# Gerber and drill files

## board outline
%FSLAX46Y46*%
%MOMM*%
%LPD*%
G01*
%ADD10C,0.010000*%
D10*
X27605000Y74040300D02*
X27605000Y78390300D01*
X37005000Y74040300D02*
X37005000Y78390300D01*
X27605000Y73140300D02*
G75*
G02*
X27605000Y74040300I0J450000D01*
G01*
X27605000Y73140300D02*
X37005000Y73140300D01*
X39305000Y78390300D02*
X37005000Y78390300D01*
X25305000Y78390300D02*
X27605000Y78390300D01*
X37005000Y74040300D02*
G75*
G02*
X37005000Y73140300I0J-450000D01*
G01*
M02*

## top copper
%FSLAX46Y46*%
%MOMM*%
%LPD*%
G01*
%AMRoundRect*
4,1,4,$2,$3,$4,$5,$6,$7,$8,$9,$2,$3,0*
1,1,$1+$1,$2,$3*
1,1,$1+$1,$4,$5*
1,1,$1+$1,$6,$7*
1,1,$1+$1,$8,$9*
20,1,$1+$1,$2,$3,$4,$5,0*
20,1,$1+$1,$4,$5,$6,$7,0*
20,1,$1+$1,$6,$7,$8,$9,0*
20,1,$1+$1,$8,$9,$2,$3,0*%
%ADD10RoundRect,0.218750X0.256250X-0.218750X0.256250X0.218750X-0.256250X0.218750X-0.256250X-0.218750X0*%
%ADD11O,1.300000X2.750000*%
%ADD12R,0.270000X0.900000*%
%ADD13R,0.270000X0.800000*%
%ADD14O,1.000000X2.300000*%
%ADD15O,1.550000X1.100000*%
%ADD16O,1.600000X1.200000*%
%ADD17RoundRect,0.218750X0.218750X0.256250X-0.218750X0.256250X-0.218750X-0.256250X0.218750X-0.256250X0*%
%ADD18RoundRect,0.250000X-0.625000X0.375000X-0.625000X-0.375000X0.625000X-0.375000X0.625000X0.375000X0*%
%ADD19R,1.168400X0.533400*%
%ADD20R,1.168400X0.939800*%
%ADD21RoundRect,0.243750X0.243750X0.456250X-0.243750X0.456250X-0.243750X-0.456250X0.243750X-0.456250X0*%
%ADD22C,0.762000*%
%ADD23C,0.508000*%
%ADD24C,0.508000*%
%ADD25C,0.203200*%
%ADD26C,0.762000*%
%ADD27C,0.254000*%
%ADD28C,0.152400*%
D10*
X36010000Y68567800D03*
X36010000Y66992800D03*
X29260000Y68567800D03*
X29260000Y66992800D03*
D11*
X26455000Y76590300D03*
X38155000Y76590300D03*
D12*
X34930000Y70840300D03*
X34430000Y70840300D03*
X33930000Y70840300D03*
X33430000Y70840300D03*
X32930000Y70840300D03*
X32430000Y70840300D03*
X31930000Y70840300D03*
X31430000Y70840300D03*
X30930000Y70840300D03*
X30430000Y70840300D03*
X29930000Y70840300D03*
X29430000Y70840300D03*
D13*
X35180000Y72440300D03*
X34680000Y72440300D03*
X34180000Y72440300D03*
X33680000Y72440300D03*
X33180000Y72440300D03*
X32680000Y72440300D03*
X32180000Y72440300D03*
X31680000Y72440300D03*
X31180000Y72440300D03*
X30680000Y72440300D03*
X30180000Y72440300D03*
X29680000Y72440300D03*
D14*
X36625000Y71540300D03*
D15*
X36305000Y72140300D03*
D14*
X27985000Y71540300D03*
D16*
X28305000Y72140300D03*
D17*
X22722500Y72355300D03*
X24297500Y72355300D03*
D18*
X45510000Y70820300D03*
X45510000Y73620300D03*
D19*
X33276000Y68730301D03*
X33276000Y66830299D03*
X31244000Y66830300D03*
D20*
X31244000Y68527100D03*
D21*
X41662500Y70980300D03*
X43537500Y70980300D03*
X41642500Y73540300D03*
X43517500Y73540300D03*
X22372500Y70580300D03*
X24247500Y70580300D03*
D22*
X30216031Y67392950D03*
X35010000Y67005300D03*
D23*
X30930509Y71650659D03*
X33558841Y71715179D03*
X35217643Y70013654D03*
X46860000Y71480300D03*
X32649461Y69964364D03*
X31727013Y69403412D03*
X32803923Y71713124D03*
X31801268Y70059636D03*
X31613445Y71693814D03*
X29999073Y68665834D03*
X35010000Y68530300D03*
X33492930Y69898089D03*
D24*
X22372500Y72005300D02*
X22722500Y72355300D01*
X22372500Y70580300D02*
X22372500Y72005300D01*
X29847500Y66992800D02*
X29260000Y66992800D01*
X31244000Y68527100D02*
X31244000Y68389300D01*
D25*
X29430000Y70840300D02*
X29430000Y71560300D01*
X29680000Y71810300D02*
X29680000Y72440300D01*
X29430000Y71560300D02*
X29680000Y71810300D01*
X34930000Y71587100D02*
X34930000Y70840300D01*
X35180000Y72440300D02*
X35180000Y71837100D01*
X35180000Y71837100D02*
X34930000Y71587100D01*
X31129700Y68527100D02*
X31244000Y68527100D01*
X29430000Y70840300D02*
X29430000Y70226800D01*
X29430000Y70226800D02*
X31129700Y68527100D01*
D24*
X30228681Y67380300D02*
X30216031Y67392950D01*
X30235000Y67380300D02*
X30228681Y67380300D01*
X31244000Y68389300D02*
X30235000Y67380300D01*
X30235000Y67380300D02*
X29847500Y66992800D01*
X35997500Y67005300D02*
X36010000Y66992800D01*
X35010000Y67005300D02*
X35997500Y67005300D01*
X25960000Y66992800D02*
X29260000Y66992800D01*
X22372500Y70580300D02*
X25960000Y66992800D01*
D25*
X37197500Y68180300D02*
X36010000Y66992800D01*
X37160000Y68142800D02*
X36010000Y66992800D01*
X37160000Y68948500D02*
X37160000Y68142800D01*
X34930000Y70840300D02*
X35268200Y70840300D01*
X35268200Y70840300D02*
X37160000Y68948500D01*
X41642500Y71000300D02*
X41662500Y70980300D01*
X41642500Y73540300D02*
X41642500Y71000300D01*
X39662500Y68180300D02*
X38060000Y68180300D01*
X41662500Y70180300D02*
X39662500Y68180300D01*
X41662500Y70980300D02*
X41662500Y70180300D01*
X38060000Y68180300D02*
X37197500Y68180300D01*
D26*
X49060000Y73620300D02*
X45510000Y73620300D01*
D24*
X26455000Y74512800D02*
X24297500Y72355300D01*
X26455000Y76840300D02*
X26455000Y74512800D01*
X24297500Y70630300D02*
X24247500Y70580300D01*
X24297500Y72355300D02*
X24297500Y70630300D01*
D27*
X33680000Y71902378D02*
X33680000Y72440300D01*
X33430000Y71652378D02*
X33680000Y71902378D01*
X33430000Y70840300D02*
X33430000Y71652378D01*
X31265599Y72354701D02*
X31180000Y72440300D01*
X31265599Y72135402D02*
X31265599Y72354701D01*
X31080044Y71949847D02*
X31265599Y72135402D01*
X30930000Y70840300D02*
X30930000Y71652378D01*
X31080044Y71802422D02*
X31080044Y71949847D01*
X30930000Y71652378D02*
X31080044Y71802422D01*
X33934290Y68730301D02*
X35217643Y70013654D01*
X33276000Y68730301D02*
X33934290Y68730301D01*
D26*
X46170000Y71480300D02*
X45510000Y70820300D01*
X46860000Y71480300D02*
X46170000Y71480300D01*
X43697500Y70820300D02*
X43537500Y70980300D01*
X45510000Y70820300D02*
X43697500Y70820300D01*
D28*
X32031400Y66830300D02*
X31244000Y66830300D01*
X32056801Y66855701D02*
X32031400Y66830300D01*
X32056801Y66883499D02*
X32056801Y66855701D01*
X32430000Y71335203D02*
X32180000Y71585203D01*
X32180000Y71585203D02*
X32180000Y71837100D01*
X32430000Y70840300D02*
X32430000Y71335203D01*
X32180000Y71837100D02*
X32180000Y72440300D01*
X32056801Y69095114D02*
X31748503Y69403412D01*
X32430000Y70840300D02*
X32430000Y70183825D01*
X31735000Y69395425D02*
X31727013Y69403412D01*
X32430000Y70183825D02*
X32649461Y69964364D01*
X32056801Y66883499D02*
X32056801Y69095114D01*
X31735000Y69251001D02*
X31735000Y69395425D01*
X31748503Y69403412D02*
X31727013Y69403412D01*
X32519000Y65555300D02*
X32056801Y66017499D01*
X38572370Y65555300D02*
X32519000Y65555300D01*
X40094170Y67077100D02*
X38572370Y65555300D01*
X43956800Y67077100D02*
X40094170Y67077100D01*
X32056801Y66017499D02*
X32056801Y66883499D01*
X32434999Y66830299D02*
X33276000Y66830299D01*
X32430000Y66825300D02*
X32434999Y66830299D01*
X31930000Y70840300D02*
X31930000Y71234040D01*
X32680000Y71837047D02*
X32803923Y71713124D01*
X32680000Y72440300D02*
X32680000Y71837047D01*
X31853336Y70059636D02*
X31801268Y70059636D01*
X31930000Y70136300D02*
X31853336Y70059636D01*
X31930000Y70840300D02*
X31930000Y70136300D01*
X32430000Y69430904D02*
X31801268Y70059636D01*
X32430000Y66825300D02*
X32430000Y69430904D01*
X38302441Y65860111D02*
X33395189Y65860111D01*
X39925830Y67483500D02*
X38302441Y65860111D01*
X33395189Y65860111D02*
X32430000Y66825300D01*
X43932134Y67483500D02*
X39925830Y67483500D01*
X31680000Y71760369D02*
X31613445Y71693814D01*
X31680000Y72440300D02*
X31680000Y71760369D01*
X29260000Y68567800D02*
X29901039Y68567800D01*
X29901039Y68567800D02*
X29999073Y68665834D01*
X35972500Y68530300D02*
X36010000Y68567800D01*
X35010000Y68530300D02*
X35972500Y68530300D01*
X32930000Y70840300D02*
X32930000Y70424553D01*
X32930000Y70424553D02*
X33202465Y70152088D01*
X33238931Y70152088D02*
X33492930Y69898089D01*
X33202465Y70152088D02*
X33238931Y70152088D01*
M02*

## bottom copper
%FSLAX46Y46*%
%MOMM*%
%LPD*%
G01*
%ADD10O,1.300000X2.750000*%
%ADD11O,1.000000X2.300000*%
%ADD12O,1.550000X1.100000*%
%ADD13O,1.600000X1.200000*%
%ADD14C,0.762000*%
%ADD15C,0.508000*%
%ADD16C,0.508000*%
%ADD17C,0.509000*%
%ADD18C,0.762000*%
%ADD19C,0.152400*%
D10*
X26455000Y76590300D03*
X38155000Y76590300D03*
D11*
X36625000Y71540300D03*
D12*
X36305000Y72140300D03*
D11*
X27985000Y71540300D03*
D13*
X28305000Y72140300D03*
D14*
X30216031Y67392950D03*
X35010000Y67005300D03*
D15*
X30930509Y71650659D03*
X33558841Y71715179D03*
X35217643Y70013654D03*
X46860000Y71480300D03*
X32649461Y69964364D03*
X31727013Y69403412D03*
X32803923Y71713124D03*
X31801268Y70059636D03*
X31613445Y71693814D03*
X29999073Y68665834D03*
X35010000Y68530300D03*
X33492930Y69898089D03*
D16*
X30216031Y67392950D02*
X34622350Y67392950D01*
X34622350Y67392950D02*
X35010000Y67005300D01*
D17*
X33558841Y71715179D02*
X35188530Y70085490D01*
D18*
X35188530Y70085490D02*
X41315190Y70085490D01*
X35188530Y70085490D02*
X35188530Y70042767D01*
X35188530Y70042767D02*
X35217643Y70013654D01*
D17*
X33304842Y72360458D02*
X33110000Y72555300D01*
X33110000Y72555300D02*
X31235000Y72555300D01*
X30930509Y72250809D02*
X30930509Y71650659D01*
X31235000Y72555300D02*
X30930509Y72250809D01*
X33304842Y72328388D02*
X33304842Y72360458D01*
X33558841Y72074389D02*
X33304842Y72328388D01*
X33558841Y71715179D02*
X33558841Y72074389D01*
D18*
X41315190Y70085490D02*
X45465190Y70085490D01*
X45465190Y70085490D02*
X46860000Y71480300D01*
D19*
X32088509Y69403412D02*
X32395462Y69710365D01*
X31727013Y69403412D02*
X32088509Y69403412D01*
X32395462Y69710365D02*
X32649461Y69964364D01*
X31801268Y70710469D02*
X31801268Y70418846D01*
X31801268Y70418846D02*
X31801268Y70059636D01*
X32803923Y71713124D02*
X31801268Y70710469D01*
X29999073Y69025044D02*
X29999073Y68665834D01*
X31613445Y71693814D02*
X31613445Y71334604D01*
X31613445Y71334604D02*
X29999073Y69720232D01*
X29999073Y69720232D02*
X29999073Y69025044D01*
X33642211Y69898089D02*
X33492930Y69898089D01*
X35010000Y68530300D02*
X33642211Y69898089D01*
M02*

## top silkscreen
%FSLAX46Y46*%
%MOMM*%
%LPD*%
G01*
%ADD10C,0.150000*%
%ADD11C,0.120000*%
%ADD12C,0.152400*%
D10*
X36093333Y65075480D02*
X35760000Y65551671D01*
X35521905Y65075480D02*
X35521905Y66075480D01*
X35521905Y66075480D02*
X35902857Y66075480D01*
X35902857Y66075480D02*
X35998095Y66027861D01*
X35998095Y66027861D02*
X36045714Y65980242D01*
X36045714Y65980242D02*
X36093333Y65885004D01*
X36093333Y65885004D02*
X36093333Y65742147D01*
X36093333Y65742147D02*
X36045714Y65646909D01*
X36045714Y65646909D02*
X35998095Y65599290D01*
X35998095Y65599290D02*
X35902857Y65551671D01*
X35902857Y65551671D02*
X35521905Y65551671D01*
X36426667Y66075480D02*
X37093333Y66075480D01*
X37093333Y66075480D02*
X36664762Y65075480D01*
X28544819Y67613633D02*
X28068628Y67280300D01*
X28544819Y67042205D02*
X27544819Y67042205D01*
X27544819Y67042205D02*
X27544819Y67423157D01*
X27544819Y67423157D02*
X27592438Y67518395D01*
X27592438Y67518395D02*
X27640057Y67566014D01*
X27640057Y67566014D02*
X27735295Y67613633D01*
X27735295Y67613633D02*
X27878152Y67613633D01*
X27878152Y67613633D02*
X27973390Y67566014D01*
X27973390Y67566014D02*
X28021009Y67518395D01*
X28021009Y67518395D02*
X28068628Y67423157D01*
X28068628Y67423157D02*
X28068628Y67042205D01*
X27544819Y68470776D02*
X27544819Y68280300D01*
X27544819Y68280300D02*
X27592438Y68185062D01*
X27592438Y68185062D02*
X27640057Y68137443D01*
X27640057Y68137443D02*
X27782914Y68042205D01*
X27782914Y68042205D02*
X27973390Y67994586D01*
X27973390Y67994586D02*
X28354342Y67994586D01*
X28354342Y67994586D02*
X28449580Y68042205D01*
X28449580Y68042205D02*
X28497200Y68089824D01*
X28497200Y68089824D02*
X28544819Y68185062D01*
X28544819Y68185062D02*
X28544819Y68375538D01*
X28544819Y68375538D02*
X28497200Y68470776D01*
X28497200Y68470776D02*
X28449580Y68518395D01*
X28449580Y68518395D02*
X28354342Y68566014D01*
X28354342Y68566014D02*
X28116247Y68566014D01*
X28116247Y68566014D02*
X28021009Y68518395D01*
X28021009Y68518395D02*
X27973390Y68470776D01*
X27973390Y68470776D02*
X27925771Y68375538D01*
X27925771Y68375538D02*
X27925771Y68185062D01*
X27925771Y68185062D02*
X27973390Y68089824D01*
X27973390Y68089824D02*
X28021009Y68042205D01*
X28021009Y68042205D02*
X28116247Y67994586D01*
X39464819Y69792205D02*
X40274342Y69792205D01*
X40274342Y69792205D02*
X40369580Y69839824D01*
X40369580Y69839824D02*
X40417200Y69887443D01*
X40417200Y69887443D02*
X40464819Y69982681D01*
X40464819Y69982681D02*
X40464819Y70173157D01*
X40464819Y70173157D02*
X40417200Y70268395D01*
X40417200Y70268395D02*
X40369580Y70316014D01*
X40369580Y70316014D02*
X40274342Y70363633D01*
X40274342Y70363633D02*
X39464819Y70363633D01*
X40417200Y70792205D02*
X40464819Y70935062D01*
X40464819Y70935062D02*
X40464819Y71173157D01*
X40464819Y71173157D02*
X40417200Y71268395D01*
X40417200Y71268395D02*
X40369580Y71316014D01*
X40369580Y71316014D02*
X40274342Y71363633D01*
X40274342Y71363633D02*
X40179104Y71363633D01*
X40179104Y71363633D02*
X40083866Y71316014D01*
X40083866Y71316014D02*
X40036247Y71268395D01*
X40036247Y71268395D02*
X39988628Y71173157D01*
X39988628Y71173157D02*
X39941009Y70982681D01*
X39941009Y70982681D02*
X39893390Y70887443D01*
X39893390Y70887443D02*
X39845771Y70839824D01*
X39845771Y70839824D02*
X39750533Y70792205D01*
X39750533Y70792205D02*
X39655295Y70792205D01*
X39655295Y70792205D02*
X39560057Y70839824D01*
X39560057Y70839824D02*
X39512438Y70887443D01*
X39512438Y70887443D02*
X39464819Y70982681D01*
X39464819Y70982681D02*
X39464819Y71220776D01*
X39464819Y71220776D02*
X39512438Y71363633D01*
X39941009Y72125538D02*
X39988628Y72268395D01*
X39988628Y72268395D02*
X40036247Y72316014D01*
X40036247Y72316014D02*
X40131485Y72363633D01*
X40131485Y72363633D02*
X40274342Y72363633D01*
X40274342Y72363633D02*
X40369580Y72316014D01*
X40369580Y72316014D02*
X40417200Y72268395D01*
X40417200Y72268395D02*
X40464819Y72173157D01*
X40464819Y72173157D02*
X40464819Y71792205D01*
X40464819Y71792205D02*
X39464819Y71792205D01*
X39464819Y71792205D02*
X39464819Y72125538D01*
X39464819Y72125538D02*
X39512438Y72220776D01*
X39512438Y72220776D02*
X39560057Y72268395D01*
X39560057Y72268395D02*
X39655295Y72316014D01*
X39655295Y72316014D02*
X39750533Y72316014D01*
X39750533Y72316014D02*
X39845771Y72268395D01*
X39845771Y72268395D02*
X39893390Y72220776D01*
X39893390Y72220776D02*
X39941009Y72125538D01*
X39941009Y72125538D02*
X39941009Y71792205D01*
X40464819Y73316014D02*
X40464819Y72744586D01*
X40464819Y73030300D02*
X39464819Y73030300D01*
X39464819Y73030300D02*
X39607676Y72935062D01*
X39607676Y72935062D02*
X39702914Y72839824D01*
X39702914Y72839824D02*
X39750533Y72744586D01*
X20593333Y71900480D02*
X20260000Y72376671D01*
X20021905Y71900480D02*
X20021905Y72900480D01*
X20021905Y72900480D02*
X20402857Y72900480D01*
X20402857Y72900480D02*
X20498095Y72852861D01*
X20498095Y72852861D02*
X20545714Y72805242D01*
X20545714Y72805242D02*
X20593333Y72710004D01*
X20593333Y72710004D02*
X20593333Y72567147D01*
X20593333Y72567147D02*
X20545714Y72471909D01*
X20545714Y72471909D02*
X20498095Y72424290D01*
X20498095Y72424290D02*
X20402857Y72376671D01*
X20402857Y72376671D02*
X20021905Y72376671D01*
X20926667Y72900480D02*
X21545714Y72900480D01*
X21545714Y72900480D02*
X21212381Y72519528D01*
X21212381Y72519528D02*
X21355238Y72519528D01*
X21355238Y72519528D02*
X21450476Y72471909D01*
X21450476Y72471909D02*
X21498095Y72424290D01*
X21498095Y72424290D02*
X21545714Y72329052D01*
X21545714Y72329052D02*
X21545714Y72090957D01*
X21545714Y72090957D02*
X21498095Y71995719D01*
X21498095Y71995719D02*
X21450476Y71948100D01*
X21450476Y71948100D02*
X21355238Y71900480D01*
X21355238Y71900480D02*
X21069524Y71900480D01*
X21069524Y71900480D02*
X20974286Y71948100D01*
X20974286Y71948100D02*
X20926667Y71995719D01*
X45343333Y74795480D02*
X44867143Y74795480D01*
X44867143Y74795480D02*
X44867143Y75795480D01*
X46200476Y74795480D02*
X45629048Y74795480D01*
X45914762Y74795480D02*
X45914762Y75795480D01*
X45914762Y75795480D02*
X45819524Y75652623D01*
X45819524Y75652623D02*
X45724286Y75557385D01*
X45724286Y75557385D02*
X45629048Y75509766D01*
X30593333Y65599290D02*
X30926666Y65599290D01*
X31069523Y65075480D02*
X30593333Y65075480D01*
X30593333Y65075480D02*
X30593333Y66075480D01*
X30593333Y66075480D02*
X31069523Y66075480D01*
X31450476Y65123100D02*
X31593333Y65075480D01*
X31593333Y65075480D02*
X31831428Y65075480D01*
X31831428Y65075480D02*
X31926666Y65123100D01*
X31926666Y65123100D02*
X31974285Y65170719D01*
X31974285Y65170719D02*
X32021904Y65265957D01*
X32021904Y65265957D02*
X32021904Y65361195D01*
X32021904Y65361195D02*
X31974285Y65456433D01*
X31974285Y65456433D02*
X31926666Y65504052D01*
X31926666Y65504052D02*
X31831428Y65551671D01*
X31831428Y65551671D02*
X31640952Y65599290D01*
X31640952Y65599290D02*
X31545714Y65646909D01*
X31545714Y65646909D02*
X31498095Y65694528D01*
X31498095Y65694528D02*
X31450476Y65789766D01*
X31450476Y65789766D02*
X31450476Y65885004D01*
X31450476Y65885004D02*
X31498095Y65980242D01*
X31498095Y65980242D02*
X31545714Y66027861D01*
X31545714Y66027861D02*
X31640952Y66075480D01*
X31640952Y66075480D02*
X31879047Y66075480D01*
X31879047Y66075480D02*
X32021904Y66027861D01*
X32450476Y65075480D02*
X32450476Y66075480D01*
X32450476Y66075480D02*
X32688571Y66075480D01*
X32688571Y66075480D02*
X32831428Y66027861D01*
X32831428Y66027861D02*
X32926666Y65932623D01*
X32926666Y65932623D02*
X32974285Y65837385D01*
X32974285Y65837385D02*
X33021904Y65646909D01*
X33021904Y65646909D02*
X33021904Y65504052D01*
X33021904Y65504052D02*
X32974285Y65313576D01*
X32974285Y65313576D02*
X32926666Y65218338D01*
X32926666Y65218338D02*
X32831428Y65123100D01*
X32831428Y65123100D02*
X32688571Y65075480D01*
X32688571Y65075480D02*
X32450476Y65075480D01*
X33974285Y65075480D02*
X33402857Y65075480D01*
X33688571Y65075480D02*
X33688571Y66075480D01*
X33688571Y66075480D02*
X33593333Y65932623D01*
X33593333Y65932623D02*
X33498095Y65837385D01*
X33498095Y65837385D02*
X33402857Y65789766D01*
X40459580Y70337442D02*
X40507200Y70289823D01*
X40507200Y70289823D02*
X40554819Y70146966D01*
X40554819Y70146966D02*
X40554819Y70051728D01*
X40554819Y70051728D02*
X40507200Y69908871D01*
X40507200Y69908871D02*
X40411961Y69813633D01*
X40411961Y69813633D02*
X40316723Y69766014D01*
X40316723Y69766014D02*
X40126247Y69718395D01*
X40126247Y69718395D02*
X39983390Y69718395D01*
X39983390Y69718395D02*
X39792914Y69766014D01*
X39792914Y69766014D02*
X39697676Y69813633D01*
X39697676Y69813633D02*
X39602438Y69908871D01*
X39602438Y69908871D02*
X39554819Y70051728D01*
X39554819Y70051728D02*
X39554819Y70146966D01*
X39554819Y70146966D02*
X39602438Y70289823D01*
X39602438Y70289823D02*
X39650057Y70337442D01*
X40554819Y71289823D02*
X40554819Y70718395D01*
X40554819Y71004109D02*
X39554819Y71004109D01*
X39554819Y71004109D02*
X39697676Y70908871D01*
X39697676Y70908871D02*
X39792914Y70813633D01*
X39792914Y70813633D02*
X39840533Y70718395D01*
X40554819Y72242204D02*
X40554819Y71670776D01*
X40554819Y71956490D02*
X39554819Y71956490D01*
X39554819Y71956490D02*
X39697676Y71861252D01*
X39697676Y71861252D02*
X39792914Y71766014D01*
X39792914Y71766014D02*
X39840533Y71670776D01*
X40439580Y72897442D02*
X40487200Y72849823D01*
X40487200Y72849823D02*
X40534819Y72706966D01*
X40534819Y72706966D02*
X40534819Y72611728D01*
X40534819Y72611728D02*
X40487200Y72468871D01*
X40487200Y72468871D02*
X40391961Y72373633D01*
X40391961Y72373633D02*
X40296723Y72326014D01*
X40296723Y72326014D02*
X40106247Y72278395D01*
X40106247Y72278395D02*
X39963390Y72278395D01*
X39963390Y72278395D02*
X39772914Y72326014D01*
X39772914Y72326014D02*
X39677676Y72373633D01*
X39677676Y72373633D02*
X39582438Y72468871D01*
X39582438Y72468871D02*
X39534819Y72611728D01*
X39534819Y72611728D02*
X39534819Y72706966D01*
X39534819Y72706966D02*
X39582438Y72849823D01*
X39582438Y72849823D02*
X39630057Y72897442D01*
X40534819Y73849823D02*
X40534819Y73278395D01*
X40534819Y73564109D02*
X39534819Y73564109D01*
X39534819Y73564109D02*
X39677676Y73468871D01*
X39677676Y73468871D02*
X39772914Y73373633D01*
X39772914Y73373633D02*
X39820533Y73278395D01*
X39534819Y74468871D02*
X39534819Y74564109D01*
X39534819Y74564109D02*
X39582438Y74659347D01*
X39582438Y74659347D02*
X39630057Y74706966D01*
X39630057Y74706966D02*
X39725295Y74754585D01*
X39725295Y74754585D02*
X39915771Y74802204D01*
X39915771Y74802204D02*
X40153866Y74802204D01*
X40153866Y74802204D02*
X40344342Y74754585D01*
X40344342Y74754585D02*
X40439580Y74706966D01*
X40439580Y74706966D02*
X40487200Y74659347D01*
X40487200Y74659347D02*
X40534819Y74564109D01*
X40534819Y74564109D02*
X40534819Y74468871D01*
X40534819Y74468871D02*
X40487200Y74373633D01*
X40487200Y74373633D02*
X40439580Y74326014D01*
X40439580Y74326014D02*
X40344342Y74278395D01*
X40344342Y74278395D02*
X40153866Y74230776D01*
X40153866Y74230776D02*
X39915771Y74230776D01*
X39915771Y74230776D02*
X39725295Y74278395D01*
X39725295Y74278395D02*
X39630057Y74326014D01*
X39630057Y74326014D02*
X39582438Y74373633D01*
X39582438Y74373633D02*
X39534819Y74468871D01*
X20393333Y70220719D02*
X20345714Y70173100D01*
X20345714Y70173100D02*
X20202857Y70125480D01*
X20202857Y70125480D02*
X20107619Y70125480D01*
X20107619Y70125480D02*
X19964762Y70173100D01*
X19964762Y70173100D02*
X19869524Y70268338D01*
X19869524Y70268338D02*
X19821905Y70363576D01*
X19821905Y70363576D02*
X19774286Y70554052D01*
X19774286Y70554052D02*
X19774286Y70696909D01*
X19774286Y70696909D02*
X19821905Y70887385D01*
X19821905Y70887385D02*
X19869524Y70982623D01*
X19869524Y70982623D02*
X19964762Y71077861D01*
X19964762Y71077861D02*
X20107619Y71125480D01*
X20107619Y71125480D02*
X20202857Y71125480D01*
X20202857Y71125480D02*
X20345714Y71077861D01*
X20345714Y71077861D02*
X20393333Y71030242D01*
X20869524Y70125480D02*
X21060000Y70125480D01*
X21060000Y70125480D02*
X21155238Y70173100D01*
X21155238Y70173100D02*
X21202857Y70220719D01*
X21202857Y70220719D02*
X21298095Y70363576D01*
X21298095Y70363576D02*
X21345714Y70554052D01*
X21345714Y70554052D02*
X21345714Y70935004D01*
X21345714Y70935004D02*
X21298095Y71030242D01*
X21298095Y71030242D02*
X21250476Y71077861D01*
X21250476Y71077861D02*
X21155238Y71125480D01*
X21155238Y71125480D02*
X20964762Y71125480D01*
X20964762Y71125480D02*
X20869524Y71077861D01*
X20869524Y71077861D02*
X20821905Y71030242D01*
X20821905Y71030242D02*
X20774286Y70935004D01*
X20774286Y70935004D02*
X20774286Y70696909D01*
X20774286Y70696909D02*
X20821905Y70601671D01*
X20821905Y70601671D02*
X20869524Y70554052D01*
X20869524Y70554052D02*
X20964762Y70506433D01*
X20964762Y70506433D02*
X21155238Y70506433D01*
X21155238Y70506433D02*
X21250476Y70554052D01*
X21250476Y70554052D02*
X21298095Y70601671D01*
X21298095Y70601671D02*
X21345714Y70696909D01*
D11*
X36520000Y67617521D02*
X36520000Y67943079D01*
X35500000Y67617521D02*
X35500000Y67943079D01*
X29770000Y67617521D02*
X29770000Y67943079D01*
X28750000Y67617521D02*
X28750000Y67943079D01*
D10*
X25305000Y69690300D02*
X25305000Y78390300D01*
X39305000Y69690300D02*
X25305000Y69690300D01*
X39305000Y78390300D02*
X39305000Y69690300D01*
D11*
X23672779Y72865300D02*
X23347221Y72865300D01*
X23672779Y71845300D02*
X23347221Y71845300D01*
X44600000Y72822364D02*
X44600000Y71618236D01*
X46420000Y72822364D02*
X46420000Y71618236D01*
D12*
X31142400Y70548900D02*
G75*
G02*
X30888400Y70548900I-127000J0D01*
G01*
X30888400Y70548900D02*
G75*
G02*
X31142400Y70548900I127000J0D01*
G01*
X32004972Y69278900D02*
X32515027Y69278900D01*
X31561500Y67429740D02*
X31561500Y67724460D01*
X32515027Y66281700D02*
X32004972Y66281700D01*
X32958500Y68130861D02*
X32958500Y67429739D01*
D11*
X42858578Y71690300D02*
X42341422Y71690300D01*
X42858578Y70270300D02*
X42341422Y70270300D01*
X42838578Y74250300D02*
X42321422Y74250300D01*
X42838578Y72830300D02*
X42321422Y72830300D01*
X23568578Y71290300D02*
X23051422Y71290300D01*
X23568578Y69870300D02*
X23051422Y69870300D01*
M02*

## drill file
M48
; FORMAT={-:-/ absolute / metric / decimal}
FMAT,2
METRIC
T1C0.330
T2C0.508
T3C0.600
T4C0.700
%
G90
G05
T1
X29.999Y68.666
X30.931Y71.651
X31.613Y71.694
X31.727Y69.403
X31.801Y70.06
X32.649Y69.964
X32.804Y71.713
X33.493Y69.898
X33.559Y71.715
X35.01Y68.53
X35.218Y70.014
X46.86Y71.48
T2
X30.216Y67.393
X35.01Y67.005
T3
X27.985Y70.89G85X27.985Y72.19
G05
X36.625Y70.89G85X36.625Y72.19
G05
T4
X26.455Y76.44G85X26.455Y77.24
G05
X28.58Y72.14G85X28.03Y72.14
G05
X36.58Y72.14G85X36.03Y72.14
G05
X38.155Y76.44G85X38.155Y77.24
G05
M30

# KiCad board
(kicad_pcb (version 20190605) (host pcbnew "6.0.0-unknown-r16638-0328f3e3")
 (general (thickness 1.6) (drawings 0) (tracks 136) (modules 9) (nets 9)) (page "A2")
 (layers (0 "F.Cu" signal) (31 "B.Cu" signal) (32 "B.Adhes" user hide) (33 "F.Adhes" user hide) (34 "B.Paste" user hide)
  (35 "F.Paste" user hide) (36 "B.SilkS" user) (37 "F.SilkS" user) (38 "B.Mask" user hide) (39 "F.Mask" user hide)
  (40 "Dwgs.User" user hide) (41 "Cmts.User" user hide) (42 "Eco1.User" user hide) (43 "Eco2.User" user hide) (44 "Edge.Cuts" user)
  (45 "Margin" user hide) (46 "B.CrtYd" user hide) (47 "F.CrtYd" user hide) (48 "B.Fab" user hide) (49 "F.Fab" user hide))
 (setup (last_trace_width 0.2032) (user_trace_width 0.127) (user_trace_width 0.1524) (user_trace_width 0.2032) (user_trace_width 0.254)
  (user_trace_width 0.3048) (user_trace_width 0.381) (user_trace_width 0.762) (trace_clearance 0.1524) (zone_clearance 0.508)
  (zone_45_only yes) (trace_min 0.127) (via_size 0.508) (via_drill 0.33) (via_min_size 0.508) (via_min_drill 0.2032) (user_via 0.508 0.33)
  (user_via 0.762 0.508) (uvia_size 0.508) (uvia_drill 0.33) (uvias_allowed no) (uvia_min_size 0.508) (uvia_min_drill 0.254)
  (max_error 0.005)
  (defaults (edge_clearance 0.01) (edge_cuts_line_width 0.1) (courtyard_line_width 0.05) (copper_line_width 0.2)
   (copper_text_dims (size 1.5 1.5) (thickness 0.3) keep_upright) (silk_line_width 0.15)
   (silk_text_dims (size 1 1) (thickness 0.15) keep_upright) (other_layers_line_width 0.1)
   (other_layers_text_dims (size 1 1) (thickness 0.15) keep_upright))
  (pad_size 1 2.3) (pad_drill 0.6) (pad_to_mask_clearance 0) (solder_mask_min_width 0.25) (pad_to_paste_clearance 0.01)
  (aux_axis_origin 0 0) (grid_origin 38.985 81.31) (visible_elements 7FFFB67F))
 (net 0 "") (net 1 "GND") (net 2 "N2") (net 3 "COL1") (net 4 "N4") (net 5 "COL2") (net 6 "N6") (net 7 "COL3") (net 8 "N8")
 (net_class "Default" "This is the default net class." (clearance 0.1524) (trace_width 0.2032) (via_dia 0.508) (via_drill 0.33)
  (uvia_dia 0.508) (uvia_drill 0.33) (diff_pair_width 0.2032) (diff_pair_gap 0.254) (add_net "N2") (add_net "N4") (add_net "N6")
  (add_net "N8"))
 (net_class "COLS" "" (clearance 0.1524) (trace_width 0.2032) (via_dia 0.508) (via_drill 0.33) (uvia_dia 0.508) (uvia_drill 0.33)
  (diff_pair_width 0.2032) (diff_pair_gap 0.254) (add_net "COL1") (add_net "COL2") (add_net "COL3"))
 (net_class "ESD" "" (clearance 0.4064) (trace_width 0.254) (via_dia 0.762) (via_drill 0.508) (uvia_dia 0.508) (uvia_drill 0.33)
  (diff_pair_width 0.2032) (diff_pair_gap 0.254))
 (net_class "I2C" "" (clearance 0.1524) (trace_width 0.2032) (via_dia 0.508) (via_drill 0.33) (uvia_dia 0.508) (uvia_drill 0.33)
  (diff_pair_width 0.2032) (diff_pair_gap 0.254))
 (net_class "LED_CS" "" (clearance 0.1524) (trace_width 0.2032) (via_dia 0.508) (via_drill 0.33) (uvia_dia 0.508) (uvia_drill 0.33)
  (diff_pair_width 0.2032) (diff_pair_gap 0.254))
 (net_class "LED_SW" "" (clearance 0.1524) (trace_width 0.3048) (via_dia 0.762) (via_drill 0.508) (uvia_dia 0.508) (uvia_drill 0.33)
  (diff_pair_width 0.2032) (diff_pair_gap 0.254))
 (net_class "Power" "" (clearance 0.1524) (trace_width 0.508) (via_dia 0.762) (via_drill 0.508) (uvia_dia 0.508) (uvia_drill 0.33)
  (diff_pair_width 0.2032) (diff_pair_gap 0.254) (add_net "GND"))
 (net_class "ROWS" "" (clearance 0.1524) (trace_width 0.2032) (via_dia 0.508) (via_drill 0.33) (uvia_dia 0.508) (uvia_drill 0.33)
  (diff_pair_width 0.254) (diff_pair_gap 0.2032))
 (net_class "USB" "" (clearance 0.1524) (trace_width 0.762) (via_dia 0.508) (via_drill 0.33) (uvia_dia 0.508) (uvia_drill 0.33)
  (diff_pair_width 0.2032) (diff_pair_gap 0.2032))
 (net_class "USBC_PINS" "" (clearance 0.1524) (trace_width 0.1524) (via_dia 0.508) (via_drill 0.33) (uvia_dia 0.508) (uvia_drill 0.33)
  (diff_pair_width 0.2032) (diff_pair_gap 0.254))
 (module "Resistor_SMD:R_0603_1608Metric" (layer "F.Cu") (at 36.01 -67.7803 90)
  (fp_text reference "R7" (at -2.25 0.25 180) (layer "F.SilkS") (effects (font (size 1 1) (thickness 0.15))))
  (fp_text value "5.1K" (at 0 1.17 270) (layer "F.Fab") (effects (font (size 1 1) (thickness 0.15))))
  (fp_line (start -0.162779 0.51) (end 0.162779 0.51) (layer "F.SilkS") (width 0.12))
  (fp_line (start -0.162779 -0.51) (end 0.162779 -0.51) (layer "F.SilkS") (width 0.12))
  (pad "2" smd roundrect (at 0.7875 0 90) (size 0.875 0.95) (layers "F.Cu" "F.Paste" "F.Mask") (roundrect_rratio 0.25))
  (pad "1" smd roundrect (at -0.7875 0 90) (size 0.875 0.95) (layers "F.Cu" "F.Paste" "F.Mask") (roundrect_rratio 0.25)))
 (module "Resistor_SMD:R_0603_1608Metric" (layer "F.Cu") (at 29.26 -67.7803 90)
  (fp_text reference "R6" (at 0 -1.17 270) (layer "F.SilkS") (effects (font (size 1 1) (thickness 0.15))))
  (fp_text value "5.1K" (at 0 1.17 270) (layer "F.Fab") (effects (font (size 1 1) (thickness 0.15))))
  (fp_line (start -0.162779 0.51) (end 0.162779 0.51) (layer "F.SilkS") (width 0.12))
  (fp_line (start -0.162779 -0.51) (end 0.162779 -0.51) (layer "F.SilkS") (width 0.12))
  (pad "2" smd roundrect (at 0.7875 0 90) (size 0.875 0.95) (layers "F.Cu" "F.Paste" "F.Mask") (roundrect_rratio 0.25))
  (pad "1" smd roundrect (at -0.7875 0 90) (size 0.875 0.95) (layers "F.Cu" "F.Paste" "F.Mask") (roundrect_rratio 0.25)))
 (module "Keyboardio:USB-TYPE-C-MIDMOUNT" (layer "F.Cu") (at 32.305 -71.5403 180) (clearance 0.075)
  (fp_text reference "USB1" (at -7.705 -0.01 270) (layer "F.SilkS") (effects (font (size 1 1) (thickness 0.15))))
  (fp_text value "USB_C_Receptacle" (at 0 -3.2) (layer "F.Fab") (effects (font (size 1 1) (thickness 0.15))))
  (fp_line (start 7 -1.85) (end 7 6.85) (layer "F.SilkS") (width 0.15))
  (fp_line (start -7 -1.85) (end 7 -1.85) (layer "F.SilkS") (width 0.15))
  (fp_line (start -7 6.85) (end -7 -1.85) (layer "F.SilkS") (width 0.15))
  (fp_line (start 4.7 2.5) (end 4.7 6.85) (layer "Edge.Cuts") (width 0.01))
  (fp_line (start -4.7 2.5) (end -4.7 6.85) (layer "Edge.Cuts") (width 0.01))
  (fp_arc (start 4.7 2.05) (end 4.7 1.6) (angle 180) (layer "Edge.Cuts") (width 0.01))
  (fp_line (start 4.7 1.6) (end -4.7 1.6) (layer "Edge.Cuts") (width 0.01))
  (fp_line (start -7 6.85) (end -4.7 6.85) (layer "Edge.Cuts") (width 0.01))
  (fp_line (start 7 6.85) (end 4.7 6.85) (layer "Edge.Cuts") (width 0.01))
  (fp_arc (start -4.7 2.05) (end -4.7 2.5) (angle 180) (layer "Edge.Cuts") (width 0.01))
  (pad "S1" thru_hole oval (at 5.85 5.3 180) (size 1.3 2.75) (drill oval 0.7 1.5 (offset 0 -0.25)) (layers *.Cu *.Mask))
  (pad "S1" thru_hole oval (at -5.85 5.3 180) (size 1.3 2.75) (drill oval 0.7 1.5 (offset 0 -0.25)) (layers *.Cu *.Mask))
  (pad "A1" smd rect (at -2.625 -0.7 180) (size 0.27 0.9) (layers "F.Cu" "F.Paste" "F.Mask"))
  (pad "A2" smd rect (at -2.125 -0.7 180) (size 0.27 0.9) (layers "F.Cu" "F.Paste" "F.Mask"))
  (pad "A3" smd rect (at -1.625 -0.7 180) (size 0.27 0.9) (layers "F.Cu" "F.Paste" "F.Mask"))
  (pad "A4" smd rect (at -1.125 -0.7 180) (size 0.27 0.9) (layers "F.Cu" "F.Paste" "F.Mask"))
  (pad "A5" smd rect (at -0.625 -0.7 180) (size 0.27 0.9) (layers "F.Cu" "F.Paste" "F.Mask"))
  (pad "A6" smd rect (at -0.125 -0.7 180) (size 0.27 0.9) (layers "F.Cu" "F.Paste" "F.Mask"))
  (pad "A7" smd rect (at 0.375 -0.7 180) (size 0.27 0.9) (layers "F.Cu" "F.Paste" "F.Mask"))
  (pad "A8" smd rect (at 0.875 -0.7 180) (size 0.27 0.9) (layers "F.Cu" "F.Paste" "F.Mask"))
  (pad "A9" smd rect (at 1.375 -0.7 180) (size 0.27 0.9) (layers "F.Cu" "F.Paste" "F.Mask"))
  (pad "A10" smd rect (at 1.875 -0.7 180) (size 0.27 0.9) (layers "F.Cu" "F.Paste" "F.Mask"))
  (pad "A11" smd rect (at 2.375 -0.7 180) (size 0.27 0.9) (layers "F.Cu" "F.Paste" "F.Mask"))
  (pad "A12" smd rect (at 2.875 -0.7 180) (size 0.27 0.9) (layers "F.Cu" "F.Adhes" "F.Paste" "F.Mask"))
  (pad "B12" smd rect (at -2.875 0.9 180) (size 0.27 0.8) (layers "F.Cu" "F.Paste" "F.Mask"))
  (pad "B11" smd rect (at -2.375 0.9 180) (size 0.27 0.8) (layers "F.Cu" "F.Paste" "F.Mask"))
  (pad "B10" smd rect (at -1.875 0.9 180) (size 0.27 0.8) (layers "F.Cu" "F.Paste" "F.Mask"))
  (pad "B9" smd rect (at -1.375 0.9 180) (size 0.27 0.8) (layers "F.Cu" "F.Paste" "F.Mask"))
  (pad "B8" smd rect (at -0.875 0.9 180) (size 0.27 0.8) (layers "F.Cu" "F.Paste" "F.Mask"))
  (pad "B7" smd rect (at -0.375 0.9 180) (size 0.27 0.8) (layers "F.Cu" "F.Paste" "F.Mask"))
  (pad "B6" smd rect (at 0.125 0.9 180) (size 0.27 0.8) (layers "F.Cu" "F.Paste" "F.Mask"))
  (pad "B5" smd rect (at 0.625 0.9 180) (size 0.27 0.8) (layers "F.Cu" "F.Paste" "F.Mask"))
  (pad "B4" smd rect (at 1.125 0.9 180) (size 0.27 0.8) (layers "F.Cu" "F.Paste" "F.Mask"))
  (pad "B3" smd rect (at 1.625 0.9 180) (size 0.27 0.8) (layers "F.Cu" "F.Paste" "F.Mask"))
  (pad "B2" smd rect (at 2.125 0.9 180) (size 0.27 0.8) (layers "F.Cu" "F.Paste" "F.Mask"))
  (pad "B1" smd rect (at 2.625 0.9 180) (size 0.27 0.8) (layers "F.Cu" "F.Paste" "F.Mask"))
  (pad "S1" thru_hole oval (at -4.32 0 180) (size 1 2.3) (drill oval 0.6 1.9) (layers *.Cu *.Mask))
  (pad "S1" thru_hole oval (at -4 0.6 180) (size 1.55 1.1) (drill oval 1.25 0.7) (layers *.Cu *.Mask))
  (pad "S1" thru_hole oval (at 4.32 0 180) (size 1 2.3) (drill oval 0.6 1.9) (layers *.Cu *.Mask))
  (pad "S1" thru_hole oval (at 4 0.6 180) (size 1.6 1.2) (drill oval 1.25 0.7) (layers *.Cu *.Mask)))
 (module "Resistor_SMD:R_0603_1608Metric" (layer "F.Cu") (at 23.51 -72.3553 180)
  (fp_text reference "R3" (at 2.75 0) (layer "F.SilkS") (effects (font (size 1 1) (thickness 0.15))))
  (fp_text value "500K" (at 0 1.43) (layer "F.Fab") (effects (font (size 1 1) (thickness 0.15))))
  (fp_line (start -0.162779 0.51) (end 0.162779 0.51) (layer "F.SilkS") (width 0.12))
  (fp_line (start -0.162779 -0.51) (end 0.162779 -0.51) (layer "F.SilkS") (width 0.12))
  (pad "2" smd roundrect (at 0.7875 0 180) (size 0.875 0.95) (layers "F.Cu" "F.Paste" "F.Mask") (roundrect_rratio 0.25))
  (pad "1" smd roundrect (at -0.7875 0 180) (size 0.875 0.95) (layers "F.Cu" "F.Paste" "F.Mask") (roundrect_rratio 0.25)))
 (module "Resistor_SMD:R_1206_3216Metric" (layer "F.Cu") (at 45.51 -72.2203 270)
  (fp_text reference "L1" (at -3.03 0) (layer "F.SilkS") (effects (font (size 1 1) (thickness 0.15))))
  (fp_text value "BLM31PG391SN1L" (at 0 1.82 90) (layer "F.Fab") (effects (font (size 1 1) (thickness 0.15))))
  (fp_line (start -0.602064 0.91) (end 0.602064 0.91) (layer "F.SilkS") (width 0.12))
  (fp_line (start -0.602064 -0.91) (end 0.602064 -0.91) (layer "F.SilkS") (width 0.12))
  (pad "2" smd roundrect (at 1.4 0 270) (size 1.25 1.75) (layers "F.Cu" "F.Paste" "F.Mask") (roundrect_rratio 0.2))
  (pad "1" smd roundrect (at -1.4 0 270) (size 1.25 1.75) (layers "F.Cu" "F.Paste" "F.Mask") (roundrect_rratio 0.2)))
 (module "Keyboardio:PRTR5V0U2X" (layer "F.Cu") (at 32.26 -67.7803 270)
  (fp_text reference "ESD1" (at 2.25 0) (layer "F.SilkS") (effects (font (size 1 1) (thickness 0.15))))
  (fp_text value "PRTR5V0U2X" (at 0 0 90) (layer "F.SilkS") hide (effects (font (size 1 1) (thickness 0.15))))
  (fp_circle (center -2.7686 1.2446) (end -2.6416 1.2446) (layer "F.SilkS") (width 0.1524))
  (fp_line (start -1.4986 0.255028) (end -1.4986 -0.255027) (layer "F.SilkS") (width 0.1524))
  (fp_line (start 0.35056 0.6985) (end 0.05584 0.6985) (layer "F.SilkS") (width 0.1524))
  (fp_line (start 1.4986 -0.255027) (end 1.4986 0.255028) (layer "F.SilkS") (width 0.1524))
  (fp_line (start -0.350561 -0.6985) (end 0.350561 -0.6985) (layer "F.SilkS") (width 0.1524))
  (pad "4" smd rect (at -0.950001 -1.016 270) (size 0.5334 1.1684) (layers "F.Cu" "F.Paste" "F.Mask"))
  (pad "3" smd rect (at 0.950001 -1.016 270) (size 0.5334 1.1684) (layers "F.Cu" "F.Paste" "F.Mask"))
  (pad "2" smd rect (at 0.95 1.016 270) (size 0.5334 1.1684) (layers "F.Cu" "F.Paste" "F.Mask"))
  (pad "1" smd rect (at -0.7468 1.016 270) (size 0.9398 1.1684) (layers "F.Cu" "F.Paste" "F.Mask")))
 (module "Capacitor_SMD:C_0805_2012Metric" (layer "F.Cu") (at 42.6 -70.9803 180)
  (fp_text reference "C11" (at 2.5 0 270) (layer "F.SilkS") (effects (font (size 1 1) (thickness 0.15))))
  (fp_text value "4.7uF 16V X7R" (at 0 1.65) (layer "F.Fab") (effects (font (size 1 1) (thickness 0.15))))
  (fp_line (start -0.258578 0.71) (end 0.258578 0.71) (layer "F.SilkS") (width 0.12))
  (fp_line (start -0.258578 -0.71) (end 0.258578 -0.71) (layer "F.SilkS") (width 0.12))
  (pad "2" smd roundrect (at 0.9375 0 180) (size 0.975 1.4) (layers "F.Cu" "F.Paste" "F.Mask") (roundrect_rratio 0.25))
  (pad "1" smd roundrect (at -0.9375 0 180) (size 0.975 1.4) (layers "F.Cu" "F.Paste" "F.Mask") (roundrect_rratio 0.25)))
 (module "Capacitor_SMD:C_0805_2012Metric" (layer "F.Cu") (at 42.58 -73.5403 180)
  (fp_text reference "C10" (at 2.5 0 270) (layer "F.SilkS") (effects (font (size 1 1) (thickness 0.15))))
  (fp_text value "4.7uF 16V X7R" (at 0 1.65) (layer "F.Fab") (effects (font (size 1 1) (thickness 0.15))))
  (fp_line (start -0.258578 0.71) (end 0.258578 0.71) (layer "F.SilkS") (width 0.12))
  (fp_line (start -0.258578 -0.71) (end 0.258578 -0.71) (layer "F.SilkS") (width 0.12))
  (pad "2" smd roundrect (at 0.9375 0 180) (size 0.975 1.4) (layers "F.Cu" "F.Paste" "F.Mask") (roundrect_rratio 0.25))
  (pad "1" smd roundrect (at -0.9375 0 180) (size 0.975 1.4) (layers "F.Cu" "F.Paste" "F.Mask") (roundrect_rratio 0.25)))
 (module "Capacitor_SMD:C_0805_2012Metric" (layer "F.Cu") (at 23.31 -70.5803 180)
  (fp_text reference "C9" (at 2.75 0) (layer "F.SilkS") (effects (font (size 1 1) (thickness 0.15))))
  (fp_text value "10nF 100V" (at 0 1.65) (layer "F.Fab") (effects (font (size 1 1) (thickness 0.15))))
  (fp_line (start -0.258578 0.71) (end 0.258578 0.71) (layer "F.SilkS") (width 0.12))
  (fp_line (start -0.258578 -0.71) (end 0.258578 -0.71) (layer "F.SilkS") (width 0.12))
  (pad "2" smd roundrect (at 0.9375 0 180) (size 0.975 1.4) (layers "F.Cu" "F.Paste" "F.Mask") (roundrect_rratio 0.25))
  (pad "1" smd roundrect (at -0.9375 0 180) (size 0.975 1.4) (layers "F.Cu" "F.Paste" "F.Mask") (roundrect_rratio 0.25)))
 (segment (start 22.3725 -72.0053) (end 22.7225 -72.3553) (width 0.508) (layer "F.Cu") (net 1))
 (segment (start 22.3725 -70.5803) (end 22.3725 -72.0053) (width 0.508) (layer "F.Cu") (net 1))
 (segment (start 29.8475 -66.9928) (end 29.26 -66.9928) (width 0.508) (layer "F.Cu") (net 1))
 (segment (start 31.244 -68.5271) (end 31.244 -68.3893) (width 0.508) (layer "F.Cu") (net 1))
 (segment (start 29.43 -70.8403) (end 29.43 -71.5603) (width 0.2032) (layer "F.Cu") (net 1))
 (segment (start 29.68 -71.8103) (end 29.68 -72.4403) (width 0.2032) (layer "F.Cu") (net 1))
 (segment (start 29.43 -71.5603) (end 29.68 -71.8103) (width 0.2032) (layer "F.Cu") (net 1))
 (segment (start 34.93 -71.5871) (end 34.93 -70.8403) (width 0.2032) (layer "F.Cu") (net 1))
 (segment (start 35.18 -72.4403) (end 35.18 -71.8371) (width 0.2032) (layer "F.Cu") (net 1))
 (segment (start 35.18 -71.8371) (end 34.93 -71.5871) (width 0.2032) (layer "F.Cu") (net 1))
 (segment (start 31.1297 -68.5271) (end 31.244 -68.5271) (width 0.2032) (layer "F.Cu") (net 1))
 (segment (start 29.43 -70.8403) (end 29.43 -70.2268) (width 0.2032) (layer "F.Cu") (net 1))
 (segment (start 29.43 -70.2268) (end 31.1297 -68.5271) (width 0.2032) (layer "F.Cu") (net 1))
 (via (at 30.216031 -67.39295) (size 0.762) (drill 0.508) (layers "F.Cu" "B.Cu") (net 1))
 (segment (start 30.228681 -67.3803) (end 30.216031 -67.39295) (width 0.508) (layer "F.Cu") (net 1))
 (segment (start 30.235 -67.3803) (end 30.228681 -67.3803) (width 0.508) (layer "F.Cu") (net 1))
 (segment (start 31.244 -68.3893) (end 30.235 -67.3803) (width 0.508) (layer "F.Cu") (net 1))
 (segment (start 30.235 -67.3803) (end 29.8475 -66.9928) (width 0.508) (layer "F.Cu") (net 1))
 (via (at 35.01 -67.0053) (size 0.762) (drill 0.508) (layers "F.Cu" "B.Cu") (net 1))
 (segment (start 30.216031 -67.39295) (end 34.62235 -67.39295) (width 0.508) (layer "B.Cu") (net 1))
 (segment (start 34.62235 -67.39295) (end 35.01 -67.0053) (width 0.508) (layer "B.Cu") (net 1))
 (segment (start 35.9975 -67.0053) (end 36.01 -66.9928) (width 0.508) (layer "F.Cu") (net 1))
 (segment (start 35.01 -67.0053) (end 35.9975 -67.0053) (width 0.508) (layer "F.Cu") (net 1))
 (segment (start 25.96 -66.9928) (end 29.26 -66.9928) (width 0.508) (layer "F.Cu") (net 1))
 (segment (start 22.3725 -70.5803) (end 25.96 -66.9928) (width 0.508) (layer "F.Cu") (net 1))
 (segment (start 37.1975 -68.1803) (end 36.01 -66.9928) (width 0.2032) (layer "F.Cu") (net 1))
 (segment (start 37.16 -68.1428) (end 36.01 -66.9928) (width 0.2032) (layer "F.Cu") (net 1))
 (segment (start 37.16 -68.9485) (end 37.16 -68.1428) (width 0.2032) (layer "F.Cu") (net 1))
 (segment (start 34.93 -70.8403) (end 35.2682 -70.8403) (width 0.2032) (layer "F.Cu") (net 1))
 (segment (start 35.2682 -70.8403) (end 37.16 -68.9485) (width 0.2032) (layer "F.Cu") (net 1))
 (segment (start 41.6425 -71.0003) (end 41.6625 -70.9803) (width 0.2032) (layer "F.Cu") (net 1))
 (segment (start 41.6425 -73.5403) (end 41.6425 -71.0003) (width 0.2032) (layer "F.Cu") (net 1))
 (segment (start 39.6625 -68.1803) (end 38.06 -68.1803) (width 0.2032) (layer "F.Cu") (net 1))
 (segment (start 41.6625 -70.1803) (end 39.6625 -68.1803) (width 0.2032) (layer "F.Cu") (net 1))
 (segment (start 41.6625 -70.9803) (end 41.6625 -70.1803) (width 0.2032) (layer "F.Cu") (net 1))
 (segment (start 38.06 -68.1803) (end 37.1975 -68.1803) (width 0.2032) (layer "F.Cu") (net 1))
 (segment (start 49.06 -73.6203) (end 45.51 -73.6203) (width 0.762) (layer "F.Cu") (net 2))
 (segment (start 26.455 -74.5128) (end 24.2975 -72.3553) (width 0.508) (layer "F.Cu") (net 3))
 (segment (start 26.455 -76.8403) (end 26.455 -74.5128) (width 0.508) (layer "F.Cu") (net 3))
 (segment (start 24.2975 -70.6303) (end 24.2475 -70.5803) (width 0.508) (layer "F.Cu") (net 3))
 (segment (start 24.2975 -72.3553) (end 24.2975 -70.6303) (width 0.508) (layer "F.Cu") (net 3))
 (segment (start 33.68 -71.902378) (end 33.68 -72.4403) (width 0.254) (layer "F.Cu") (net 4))
 (segment (start 33.43 -71.652378) (end 33.68 -71.902378) (width 0.254) (layer "F.Cu") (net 4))
 (segment (start 33.43 -70.8403) (end 33.43 -71.652378) (width 0.254) (layer "F.Cu") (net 4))
 (segment (start 31.265599 -72.354701) (end 31.18 -72.4403) (width 0.254) (layer "F.Cu") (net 4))
 (segment (start 31.265599 -72.135402) (end 31.265599 -72.354701) (width 0.254) (layer "F.Cu") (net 4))
 (segment (start 31.080044 -71.949847) (end 31.265599 -72.135402) (width 0.254) (layer "F.Cu") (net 4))
 (segment (start 30.93 -70.8403) (end 30.93 -71.652378) (width 0.254) (layer "F.Cu") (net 4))
 (segment (start 31.080044 -71.802422) (end 31.080044 -71.949847) (width 0.254) (layer "F.Cu") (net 4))
 (segment (start 30.93 -71.652378) (end 31.080044 -71.802422) (width 0.254) (layer "F.Cu") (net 4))
 (via (at 30.930509 -71.650659) (size 0.508) (drill 0.33) (layers "F.Cu" "B.Cu") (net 4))
 (via (at 33.558841 -71.715179) (size 0.508) (drill 0.33) (layers "F.Cu" "B.Cu") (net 4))
 (segment (start 33.558841 -71.715179) (end 35.18853 -70.08549) (width 0.509) (layer "B.Cu") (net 4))
 (segment (start 35.18853 -70.08549) (end 41.31519 -70.08549) (width 0.762) (layer "B.Cu") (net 4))
 (via (at 35.217643 -70.013654) (size 0.508) (drill 0.33) (layers "F.Cu" "B.Cu") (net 4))
 (segment (start 35.18853 -70.08549) (end 35.18853 -70.042767) (width 0.762) (layer "B.Cu") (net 4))
 (segment (start 35.18853 -70.042767) (end 35.217643 -70.013654) (width 0.762) (layer "B.Cu") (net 4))
 (segment (start 33.93429 -68.730301) (end 35.217643 -70.013654) (width 0.254) (layer "F.Cu") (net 4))
 (segment (start 33.276 -68.730301) (end 33.93429 -68.730301) (width 0.254) (layer "F.Cu") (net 4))
 (segment (start 33.304842 -72.360458) (end 33.11 -72.5553) (width 0.509) (layer "B.Cu") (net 4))
 (segment (start 33.11 -72.5553) (end 31.235 -72.5553) (width 0.509) (layer "B.Cu") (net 4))
 (segment (start 30.930509 -72.250809) (end 30.930509 -71.650659) (width 0.509) (layer "B.Cu") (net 4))
 (segment (start 31.235 -72.5553) (end 30.930509 -72.250809) (width 0.509) (layer "B.Cu") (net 4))
 (segment (start 33.304842 -72.328388) (end 33.304842 -72.360458) (width 0.509) (layer "B.Cu") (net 4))
 (segment (start 33.558841 -72.074389) (end 33.304842 -72.328388) (width 0.509) (layer "B.Cu") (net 4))
 (segment (start 33.558841 -71.715179) (end 33.558841 -72.074389) (width 0.509) (layer "B.Cu") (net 4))
 (via (at 46.86 -71.4803) (size 0.508) (drill 0.33) (layers "F.Cu" "B.Cu") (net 4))
 (segment (start 41.31519 -70.08549) (end 45.46519 -70.08549) (width 0.762) (layer "B.Cu") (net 4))
 (segment (start 45.46519 -70.08549) (end 46.86 -71.4803) (width 0.762) (layer "B.Cu") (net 4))
 (segment (start 46.17 -71.4803) (end 45.51 -70.8203) (width 0.762) (layer "F.Cu") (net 4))
 (segment (start 46.86 -71.4803) (end 46.17 -71.4803) (width 0.762) (layer "F.Cu") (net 4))
 (segment (start 43.6975 -70.8203) (end 43.5375 -70.9803) (width 0.762) (layer "F.Cu") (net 4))
 (segment (start 45.51 -70.8203) (end 43.6975 -70.8203) (width 0.762) (layer "F.Cu") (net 4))
 (segment (start 32.0314 -66.8303) (end 31.244 -66.8303) (width 0.1524) (layer "F.Cu") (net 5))
 (segment (start 32.056801 -66.855701) (end 32.0314 -66.8303) (width 0.1524) (layer "F.Cu") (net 5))
 (segment (start 32.056801 -66.883499) (end 32.056801 -66.855701) (width 0.1524) (layer "F.Cu") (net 5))
 (segment (start 32.43 -71.335203) (end 32.18 -71.585203) (width 0.1524) (layer "F.Cu") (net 5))
 (segment (start 32.18 -71.585203) (end 32.18 -71.8371) (width 0.1524) (layer "F.Cu") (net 5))
 (segment (start 32.43 -70.8403) (end 32.43 -71.335203) (width 0.1524) (layer "F.Cu") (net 5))
 (segment (start 32.18 -71.8371) (end 32.18 -72.4403) (width 0.1524) (layer "F.Cu") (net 5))
 (segment (start 32.056801 -69.095114) (end 31.748503 -69.403412) (width 0.1524) (layer "F.Cu") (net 5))
 (via (at 32.649461 -69.964364) (size 0.508) (drill 0.33) (layers "F.Cu" "B.Cu") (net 5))
 (segment (start 32.43 -70.8403) (end 32.43 -70.183825) (width 0.1524) (layer "F.Cu") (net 5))
 (segment (start 31.735 -69.395425) (end 31.727013 -69.403412) (width 0.1524) (layer "F.Cu") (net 5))
 (segment (start 32.088509 -69.403412) (end 32.395462 -69.710365) (width 0.1524) (layer "B.Cu") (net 5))
 (segment (start 32.43 -70.183825) (end 32.649461 -69.964364) (width 0.1524) (layer "F.Cu") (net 5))
 (segment (start 32.056801 -66.883499) (end 32.056801 -69.095114) (width 0.1524) (layer "F.Cu") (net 5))
 (segment (start 31.727013 -69.403412) (end 32.088509 -69.403412) (width 0.1524) (layer "B.Cu") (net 5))
 (segment (start 32.395462 -69.710365) (end 32.649461 -69.964364) (width 0.1524) (layer "B.Cu") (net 5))
 (via (at 31.727013 -69.403412) (size 0.508) (drill 0.33) (layers "F.Cu" "B.Cu") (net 5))
 (segment (start 31.735 -69.251001) (end 31.735 -69.395425) (width 0.1524) (layer "F.Cu") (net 5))
 (segment (start 31.748503 -69.403412) (end 31.727013 -69.403412) (width 0.1524) (layer "F.Cu") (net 5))
 (segment (start 32.519 -65.5553) (end 32.056801 -66.017499) (width 0.1524) (layer "F.Cu") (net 5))
 (segment (start 38.57237 -65.5553) (end 32.519 -65.5553) (width 0.1524) (layer "F.Cu") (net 5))
 (segment (start 40.09417 -67.0771) (end 38.57237 -65.5553) (width 0.1524) (layer "F.Cu") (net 5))
 (segment (start 43.9568 -67.0771) (end 40.09417 -67.0771) (width 0.1524) (layer "F.Cu") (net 5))
 (segment (start 32.056801 -66.017499) (end 32.056801 -66.883499) (width 0.1524) (layer "F.Cu") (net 5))
 (segment (start 32.434999 -66.830299) (end 33.276 -66.830299) (width 0.1524) (layer "F.Cu") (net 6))
 (segment (start 32.43 -66.8253) (end 32.434999 -66.830299) (width 0.1524) (layer "F.Cu") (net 6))
 (segment (start 31.93 -70.8403) (end 31.93 -71.23404) (width 0.1524) (layer "F.Cu") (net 6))
 (via (at 32.803923 -71.713124) (size 0.508) (drill 0.33) (layers "F.Cu" "B.Cu") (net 6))
 (segment (start 32.68 -71.837047) (end 32.803923 -71.713124) (width 0.1524) (layer "F.Cu") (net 6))
 (segment (start 32.68 -72.4403) (end 32.68 -71.837047) (width 0.1524) (layer "F.Cu") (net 6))
 (segment (start 31.801268 -70.710469) (end 31.801268 -70.418846) (width 0.1524) (layer "B.Cu") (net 6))
 (segment (start 31.801268 -70.418846) (end 31.801268 -70.059636) (width 0.1524) (layer "B.Cu") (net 6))
 (segment (start 31.853336 -70.059636) (end 31.801268 -70.059636) (width 0.1524) (layer "F.Cu") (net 6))
 (segment (start 32.803923 -71.713124) (end 31.801268 -70.710469) (width 0.1524) (layer "B.Cu") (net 6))
 (segment (start 31.93 -70.1363) (end 31.853336 -70.059636) (width 0.1524) (layer "F.Cu") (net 6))
 (via (at 31.801268 -70.059636) (size 0.508) (drill 0.33) (layers "F.Cu" "B.Cu") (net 6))
 (segment (start 31.93 -70.8403) (end 31.93 -70.1363) (width 0.1524) (layer "F.Cu") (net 6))
 (segment (start 32.43 -69.430904) (end 31.801268 -70.059636) (width 0.1524) (layer "F.Cu") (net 6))
 (segment (start 32.43 -66.8253) (end 32.43 -69.430904) (width 0.1524) (layer "F.Cu") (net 6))
 (segment (start 38.302441 -65.860111) (end 33.395189 -65.860111) (width 0.1524) (layer "F.Cu") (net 6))
 (segment (start 39.92583 -67.4835) (end 38.302441 -65.860111) (width 0.1524) (layer "F.Cu") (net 6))
 (segment (start 33.395189 -65.860111) (end 32.43 -66.8253) (width 0.1524) (layer "F.Cu") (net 6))
 (segment (start 43.932134 -67.4835) (end 39.92583 -67.4835) (width 0.1524) (layer "F.Cu") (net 6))
 (via (at 31.613445 -71.693814) (size 0.508) (drill 0.33) (layers "F.Cu" "B.Cu") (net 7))
 (segment (start 31.68 -71.760369) (end 31.613445 -71.693814) (width 0.1524) (layer "F.Cu") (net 7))
 (segment (start 31.68 -72.4403) (end 31.68 -71.760369) (width 0.1524) (layer "F.Cu") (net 7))
 (segment (start 29.999073 -69.025044) (end 29.999073 -68.665834) (width 0.1524) (layer "B.Cu") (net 7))
 (segment (start 31.613445 -71.693814) (end 31.613445 -71.334604) (width 0.1524) (layer "B.Cu") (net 7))
 (segment (start 31.613445 -71.334604) (end 29.999073 -69.720232) (width 0.1524) (layer "B.Cu") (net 7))
 (segment (start 29.26 -68.5678) (end 29.901039 -68.5678) (width 0.1524) (layer "F.Cu") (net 7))
 (via (at 29.999073 -68.665834) (size 0.508) (drill 0.33) (layers "F.Cu" "B.Cu") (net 7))
 (segment (start 29.901039 -68.5678) (end 29.999073 -68.665834) (width 0.1524) (layer "F.Cu") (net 7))
 (segment (start 29.999073 -69.720232) (end 29.999073 -69.025044) (width 0.1524) (layer "B.Cu") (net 7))
 (via (at 35.01 -68.5303) (size 0.508) (drill 0.33) (layers "F.Cu" "B.Cu") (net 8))
 (segment (start 35.9725 -68.5303) (end 36.01 -68.5678) (width 0.1524) (layer "F.Cu") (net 8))
 (segment (start 35.01 -68.5303) (end 35.9725 -68.5303) (width 0.1524) (layer "F.Cu") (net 8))
 (via (at 33.49293 -69.898089) (size 0.508) (drill 0.33) (layers "F.Cu" "B.Cu") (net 8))
 (segment (start 32.93 -70.8403) (end 32.93 -70.424553) (width 0.1524) (layer "F.Cu") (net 8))
 (segment (start 33.642211 -69.898089) (end 33.49293 -69.898089) (width 0.1524) (layer "B.Cu") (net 8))
 (segment (start 32.93 -70.424553) (end 33.202465 -70.152088) (width 0.1524) (layer "F.Cu") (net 8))
 (segment (start 33.238931 -70.152088) (end 33.49293 -69.898089) (width 0.1524) (layer "F.Cu") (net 8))
 (segment (start 33.202465 -70.152088) (end 33.238931 -70.152088) (width 0.1524) (layer "F.Cu") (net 8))
 (segment (start 35.01 -68.5303) (end 33.642211 -69.898089) (width 0.1524) (layer "B.Cu") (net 8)))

